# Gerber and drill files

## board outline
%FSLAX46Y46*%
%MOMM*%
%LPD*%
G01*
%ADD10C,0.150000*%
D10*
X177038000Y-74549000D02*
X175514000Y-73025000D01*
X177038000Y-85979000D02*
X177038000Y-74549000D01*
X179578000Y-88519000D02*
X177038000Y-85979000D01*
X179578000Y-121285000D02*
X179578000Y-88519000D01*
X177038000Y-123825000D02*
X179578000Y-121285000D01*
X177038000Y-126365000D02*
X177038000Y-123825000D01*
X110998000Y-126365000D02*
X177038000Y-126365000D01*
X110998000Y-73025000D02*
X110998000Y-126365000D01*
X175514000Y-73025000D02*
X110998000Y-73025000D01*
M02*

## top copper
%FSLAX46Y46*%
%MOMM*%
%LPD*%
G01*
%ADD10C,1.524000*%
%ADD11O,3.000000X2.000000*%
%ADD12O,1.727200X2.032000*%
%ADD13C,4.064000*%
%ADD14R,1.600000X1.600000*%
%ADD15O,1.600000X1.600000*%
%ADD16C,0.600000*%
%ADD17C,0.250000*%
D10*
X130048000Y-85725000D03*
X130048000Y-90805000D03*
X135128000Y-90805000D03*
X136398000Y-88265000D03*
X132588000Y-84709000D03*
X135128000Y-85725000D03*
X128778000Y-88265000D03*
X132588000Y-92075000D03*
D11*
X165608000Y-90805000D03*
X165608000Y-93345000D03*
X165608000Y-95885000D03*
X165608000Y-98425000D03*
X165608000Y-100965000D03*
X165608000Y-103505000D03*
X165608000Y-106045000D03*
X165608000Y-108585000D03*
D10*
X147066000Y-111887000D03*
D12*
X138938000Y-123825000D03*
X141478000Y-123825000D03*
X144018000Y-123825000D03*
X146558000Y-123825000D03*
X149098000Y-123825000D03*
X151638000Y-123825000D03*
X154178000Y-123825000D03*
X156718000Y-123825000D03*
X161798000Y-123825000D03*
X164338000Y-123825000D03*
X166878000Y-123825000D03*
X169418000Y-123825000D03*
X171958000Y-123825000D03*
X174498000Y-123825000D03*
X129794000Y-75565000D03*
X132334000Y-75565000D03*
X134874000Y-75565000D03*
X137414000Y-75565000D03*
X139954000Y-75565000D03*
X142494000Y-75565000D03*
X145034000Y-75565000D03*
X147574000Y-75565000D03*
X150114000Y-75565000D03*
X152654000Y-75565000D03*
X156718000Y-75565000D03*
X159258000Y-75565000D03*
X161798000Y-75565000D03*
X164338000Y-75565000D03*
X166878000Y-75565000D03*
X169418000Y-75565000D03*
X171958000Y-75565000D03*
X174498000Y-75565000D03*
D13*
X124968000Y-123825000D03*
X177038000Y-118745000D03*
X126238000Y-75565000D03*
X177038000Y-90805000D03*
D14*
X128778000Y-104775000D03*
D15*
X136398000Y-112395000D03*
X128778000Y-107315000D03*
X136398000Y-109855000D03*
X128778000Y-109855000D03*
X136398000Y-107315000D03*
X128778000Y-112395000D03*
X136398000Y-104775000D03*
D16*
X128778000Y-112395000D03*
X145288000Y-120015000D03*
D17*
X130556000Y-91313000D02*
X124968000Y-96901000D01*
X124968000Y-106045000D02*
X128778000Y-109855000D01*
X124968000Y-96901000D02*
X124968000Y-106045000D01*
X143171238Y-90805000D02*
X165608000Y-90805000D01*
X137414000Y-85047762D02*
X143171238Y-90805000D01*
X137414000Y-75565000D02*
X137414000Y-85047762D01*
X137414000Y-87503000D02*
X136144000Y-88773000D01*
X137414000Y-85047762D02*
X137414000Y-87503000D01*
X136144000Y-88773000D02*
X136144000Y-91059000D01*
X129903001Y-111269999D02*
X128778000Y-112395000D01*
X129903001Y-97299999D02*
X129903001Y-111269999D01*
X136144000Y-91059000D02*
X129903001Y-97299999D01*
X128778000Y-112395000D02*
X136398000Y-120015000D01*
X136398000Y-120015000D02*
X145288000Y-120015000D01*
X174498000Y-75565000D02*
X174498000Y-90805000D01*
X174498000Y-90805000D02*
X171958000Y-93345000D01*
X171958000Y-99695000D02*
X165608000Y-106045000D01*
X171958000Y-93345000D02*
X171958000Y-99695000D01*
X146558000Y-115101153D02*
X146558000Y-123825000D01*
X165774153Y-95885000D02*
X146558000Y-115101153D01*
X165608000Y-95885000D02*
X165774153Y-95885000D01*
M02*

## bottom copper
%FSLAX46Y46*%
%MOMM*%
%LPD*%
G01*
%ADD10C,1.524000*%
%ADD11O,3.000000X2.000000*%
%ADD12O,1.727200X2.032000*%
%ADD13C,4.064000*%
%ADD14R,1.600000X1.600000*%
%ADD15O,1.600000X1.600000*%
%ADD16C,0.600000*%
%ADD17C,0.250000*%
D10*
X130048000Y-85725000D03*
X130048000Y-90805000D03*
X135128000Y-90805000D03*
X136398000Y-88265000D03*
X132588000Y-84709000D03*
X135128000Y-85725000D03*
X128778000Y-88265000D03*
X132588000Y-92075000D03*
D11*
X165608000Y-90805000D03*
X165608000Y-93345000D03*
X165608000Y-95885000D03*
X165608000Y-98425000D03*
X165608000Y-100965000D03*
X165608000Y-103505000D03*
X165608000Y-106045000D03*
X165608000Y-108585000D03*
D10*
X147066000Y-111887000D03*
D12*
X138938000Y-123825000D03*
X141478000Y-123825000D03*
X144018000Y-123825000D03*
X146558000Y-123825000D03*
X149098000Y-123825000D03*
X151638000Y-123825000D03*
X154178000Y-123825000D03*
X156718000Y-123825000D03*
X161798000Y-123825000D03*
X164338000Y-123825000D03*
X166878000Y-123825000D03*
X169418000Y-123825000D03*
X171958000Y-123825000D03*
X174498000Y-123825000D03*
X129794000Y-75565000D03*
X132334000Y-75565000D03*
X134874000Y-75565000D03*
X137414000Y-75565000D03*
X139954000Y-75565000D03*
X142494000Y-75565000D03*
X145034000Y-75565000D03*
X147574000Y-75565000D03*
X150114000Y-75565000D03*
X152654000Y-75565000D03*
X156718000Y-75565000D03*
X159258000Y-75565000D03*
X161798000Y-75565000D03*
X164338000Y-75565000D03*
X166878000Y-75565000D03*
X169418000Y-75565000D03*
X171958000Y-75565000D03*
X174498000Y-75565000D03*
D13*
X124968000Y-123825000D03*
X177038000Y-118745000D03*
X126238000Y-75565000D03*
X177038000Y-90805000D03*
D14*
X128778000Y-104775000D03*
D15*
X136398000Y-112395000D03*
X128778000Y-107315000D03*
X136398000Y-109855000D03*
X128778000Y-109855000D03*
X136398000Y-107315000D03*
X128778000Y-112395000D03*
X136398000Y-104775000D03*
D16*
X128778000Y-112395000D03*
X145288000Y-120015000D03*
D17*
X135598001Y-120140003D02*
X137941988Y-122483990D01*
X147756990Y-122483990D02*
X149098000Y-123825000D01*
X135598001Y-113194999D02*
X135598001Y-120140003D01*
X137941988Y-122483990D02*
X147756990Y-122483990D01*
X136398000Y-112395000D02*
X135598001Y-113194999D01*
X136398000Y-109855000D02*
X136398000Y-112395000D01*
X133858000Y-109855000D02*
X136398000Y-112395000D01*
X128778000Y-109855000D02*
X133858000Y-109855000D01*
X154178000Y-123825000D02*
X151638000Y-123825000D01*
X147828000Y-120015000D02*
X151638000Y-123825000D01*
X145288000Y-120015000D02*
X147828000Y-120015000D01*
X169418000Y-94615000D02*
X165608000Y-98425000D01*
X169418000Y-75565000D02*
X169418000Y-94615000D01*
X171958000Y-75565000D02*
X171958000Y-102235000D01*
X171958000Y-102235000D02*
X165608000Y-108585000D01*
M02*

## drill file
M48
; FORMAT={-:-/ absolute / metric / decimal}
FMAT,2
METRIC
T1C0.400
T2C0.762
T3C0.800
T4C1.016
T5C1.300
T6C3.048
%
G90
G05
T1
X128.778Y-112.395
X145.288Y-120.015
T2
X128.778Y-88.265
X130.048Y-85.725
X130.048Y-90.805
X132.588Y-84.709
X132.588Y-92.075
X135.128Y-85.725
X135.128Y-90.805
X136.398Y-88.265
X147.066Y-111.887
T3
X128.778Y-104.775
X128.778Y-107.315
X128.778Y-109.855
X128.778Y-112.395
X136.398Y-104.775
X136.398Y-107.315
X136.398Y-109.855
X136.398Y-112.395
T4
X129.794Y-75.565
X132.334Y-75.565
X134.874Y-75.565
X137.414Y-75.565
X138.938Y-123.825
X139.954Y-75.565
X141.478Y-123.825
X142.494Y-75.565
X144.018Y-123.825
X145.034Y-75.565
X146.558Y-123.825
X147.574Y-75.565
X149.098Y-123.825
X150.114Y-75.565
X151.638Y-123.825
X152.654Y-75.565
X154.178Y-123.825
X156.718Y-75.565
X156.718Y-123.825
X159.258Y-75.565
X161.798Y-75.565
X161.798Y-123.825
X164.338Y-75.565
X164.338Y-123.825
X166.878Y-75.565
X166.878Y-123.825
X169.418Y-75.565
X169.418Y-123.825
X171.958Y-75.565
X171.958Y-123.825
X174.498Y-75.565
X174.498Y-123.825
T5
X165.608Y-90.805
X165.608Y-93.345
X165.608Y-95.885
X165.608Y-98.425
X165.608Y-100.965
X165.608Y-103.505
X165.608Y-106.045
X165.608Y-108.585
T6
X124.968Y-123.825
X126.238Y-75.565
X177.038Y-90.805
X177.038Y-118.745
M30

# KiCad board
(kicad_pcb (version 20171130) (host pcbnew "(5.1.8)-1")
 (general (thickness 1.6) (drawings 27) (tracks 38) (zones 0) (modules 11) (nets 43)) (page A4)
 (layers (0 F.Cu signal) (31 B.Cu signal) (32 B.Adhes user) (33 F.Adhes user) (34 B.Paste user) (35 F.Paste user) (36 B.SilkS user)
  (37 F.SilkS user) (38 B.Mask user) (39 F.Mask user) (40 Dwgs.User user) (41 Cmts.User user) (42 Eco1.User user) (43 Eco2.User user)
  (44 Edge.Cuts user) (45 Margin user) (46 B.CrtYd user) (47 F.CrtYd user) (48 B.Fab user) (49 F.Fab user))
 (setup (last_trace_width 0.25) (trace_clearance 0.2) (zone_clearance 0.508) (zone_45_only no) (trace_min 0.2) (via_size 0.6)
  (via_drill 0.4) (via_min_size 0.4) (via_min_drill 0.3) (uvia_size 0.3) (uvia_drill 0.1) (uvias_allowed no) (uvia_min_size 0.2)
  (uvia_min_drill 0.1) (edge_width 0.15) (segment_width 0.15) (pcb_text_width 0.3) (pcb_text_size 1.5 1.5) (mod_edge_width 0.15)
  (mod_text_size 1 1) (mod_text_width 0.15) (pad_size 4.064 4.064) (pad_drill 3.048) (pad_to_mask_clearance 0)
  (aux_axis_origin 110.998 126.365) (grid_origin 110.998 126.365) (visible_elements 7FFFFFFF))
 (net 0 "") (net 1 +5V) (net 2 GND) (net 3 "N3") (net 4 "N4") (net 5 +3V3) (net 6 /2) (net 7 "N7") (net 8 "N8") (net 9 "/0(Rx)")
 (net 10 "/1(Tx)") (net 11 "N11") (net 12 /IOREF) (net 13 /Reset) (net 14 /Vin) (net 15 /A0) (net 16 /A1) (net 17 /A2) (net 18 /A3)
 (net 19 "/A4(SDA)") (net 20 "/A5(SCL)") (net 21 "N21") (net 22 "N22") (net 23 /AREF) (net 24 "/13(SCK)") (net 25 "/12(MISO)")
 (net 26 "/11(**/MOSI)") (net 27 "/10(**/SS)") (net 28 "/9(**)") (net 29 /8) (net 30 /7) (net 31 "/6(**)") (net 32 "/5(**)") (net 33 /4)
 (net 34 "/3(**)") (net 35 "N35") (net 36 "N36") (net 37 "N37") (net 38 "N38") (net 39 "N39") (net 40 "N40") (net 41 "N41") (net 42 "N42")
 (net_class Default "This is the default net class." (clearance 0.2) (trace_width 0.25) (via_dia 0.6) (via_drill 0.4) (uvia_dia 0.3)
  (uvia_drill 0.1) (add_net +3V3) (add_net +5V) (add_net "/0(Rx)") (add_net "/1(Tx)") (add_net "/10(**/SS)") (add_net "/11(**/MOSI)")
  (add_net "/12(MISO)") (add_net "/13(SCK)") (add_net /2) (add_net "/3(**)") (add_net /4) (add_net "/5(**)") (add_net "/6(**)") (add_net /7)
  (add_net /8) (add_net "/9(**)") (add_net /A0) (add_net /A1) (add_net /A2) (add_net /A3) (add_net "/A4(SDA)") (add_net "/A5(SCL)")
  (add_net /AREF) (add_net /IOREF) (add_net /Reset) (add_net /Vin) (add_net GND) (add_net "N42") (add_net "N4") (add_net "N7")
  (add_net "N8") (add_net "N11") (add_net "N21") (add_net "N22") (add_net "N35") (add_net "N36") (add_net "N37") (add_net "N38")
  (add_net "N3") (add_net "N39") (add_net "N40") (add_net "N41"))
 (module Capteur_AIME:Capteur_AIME (layer F.Cu) (at 132.588 88.265)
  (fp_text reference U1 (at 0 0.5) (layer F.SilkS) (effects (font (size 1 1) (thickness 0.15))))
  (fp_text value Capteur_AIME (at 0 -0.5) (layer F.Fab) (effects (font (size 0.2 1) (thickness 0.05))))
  (pad 2 thru_hole circle (at -2.54 -2.54) (size 1.524 1.524) (drill 0.762) (layers *.Cu *.Mask) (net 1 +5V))
  (pad 8 thru_hole circle (at -2.54 2.54) (size 1.524 1.524) (drill 0.762) (layers *.Cu *.Mask))
  (pad 6 thru_hole circle (at 2.54 2.54) (size 1.524 1.524) (drill 0.762) (layers *.Cu *.Mask))
  (pad 5 thru_hole circle (at 3.81 0) (size 1.524 1.524) (drill 0.762) (layers *.Cu *.Mask) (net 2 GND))
  (pad 3 thru_hole circle (at 0 -3.556) (size 1.524 1.524) (drill 0.762) (layers *.Cu *.Mask) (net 1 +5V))
  (pad 4 thru_hole circle (at 2.54 -2.54) (size 1.524 1.524) (drill 0.762) (layers *.Cu *.Mask) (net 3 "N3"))
  (pad 1 thru_hole circle (at -3.81 0) (size 1.524 1.524) (drill 0.762) (layers *.Cu *.Mask))
  (pad 7 thru_hole circle (at 0 3.81) (size 1.524 1.524) (drill 0.762) (layers *.Cu *.Mask)))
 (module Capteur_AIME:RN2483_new (layer F.Cu) (at 165.608 99.695 270)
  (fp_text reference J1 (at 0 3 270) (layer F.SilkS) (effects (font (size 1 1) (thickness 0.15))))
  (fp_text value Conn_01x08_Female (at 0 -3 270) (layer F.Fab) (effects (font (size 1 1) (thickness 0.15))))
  (pad 1 thru_hole oval (at -8.89 0 270) (size 2 3) (drill 1.3) (layers *.Cu *.Mask) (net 2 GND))
  (pad 2 thru_hole oval (at -6.35 0 270) (size 2 3) (drill 1.3) (layers *.Cu *.Mask) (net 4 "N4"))
  (pad 3 thru_hole oval (at -3.81 0 270) (size 2 3) (drill 1.3) (layers *.Cu *.Mask) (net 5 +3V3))
  (pad 4 thru_hole oval (at -1.27 0 270) (size 2 3) (drill 1.3) (layers *.Cu *.Mask) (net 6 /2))
  (pad 5 thru_hole oval (at 1.27 0 270) (size 2 3) (drill 1.3) (layers *.Cu *.Mask) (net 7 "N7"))
  (pad 6 thru_hole oval (at 3.81 0 270) (size 2 3) (drill 1.3) (layers *.Cu *.Mask) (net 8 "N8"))
  (pad 7 thru_hole oval (at 6.35 0 270) (size 2 3) (drill 1.3) (layers *.Cu *.Mask) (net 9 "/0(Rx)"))
  (pad 8 thru_hole oval (at 8.89 0 270) (size 2 3) (drill 1.3) (layers *.Cu *.Mask) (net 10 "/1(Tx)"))
  (pad 9 thru_hole circle (at 12.192 18.542 270) (size 1.524 1.524) (drill 0.762) (layers *.Cu *.Mask)))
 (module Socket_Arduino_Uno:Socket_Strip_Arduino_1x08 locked (layer F.Cu) (at 138.938 123.825)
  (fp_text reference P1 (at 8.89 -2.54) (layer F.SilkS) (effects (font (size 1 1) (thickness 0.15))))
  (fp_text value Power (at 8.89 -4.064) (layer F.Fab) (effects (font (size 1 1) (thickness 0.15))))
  (pad 1 thru_hole oval (at 0 0) (size 1.7272 2.032) (drill 1.016) (layers *.Cu *.Mask F.SilkS) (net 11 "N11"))
  (pad 2 thru_hole oval (at 2.54 0) (size 1.7272 2.032) (drill 1.016) (layers *.Cu *.Mask F.SilkS) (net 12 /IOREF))
  (pad 3 thru_hole oval (at 5.08 0) (size 1.7272 2.032) (drill 1.016) (layers *.Cu *.Mask F.SilkS) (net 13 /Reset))
  (pad 4 thru_hole oval (at 7.62 0) (size 1.7272 2.032) (drill 1.016) (layers *.Cu *.Mask F.SilkS) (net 5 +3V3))
  (pad 5 thru_hole oval (at 10.16 0) (size 1.7272 2.032) (drill 1.016) (layers *.Cu *.Mask F.SilkS) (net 1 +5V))
  (pad 6 thru_hole oval (at 12.7 0) (size 1.7272 2.032) (drill 1.016) (layers *.Cu *.Mask F.SilkS) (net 2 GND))
  (pad 7 thru_hole oval (at 15.24 0) (size 1.7272 2.032) (drill 1.016) (layers *.Cu *.Mask F.SilkS) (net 2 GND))
  (pad 8 thru_hole oval (at 17.78 0) (size 1.7272 2.032) (drill 1.016) (layers *.Cu *.Mask F.SilkS) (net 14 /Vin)))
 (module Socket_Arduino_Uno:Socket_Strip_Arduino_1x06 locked (layer F.Cu) (at 161.798 123.825)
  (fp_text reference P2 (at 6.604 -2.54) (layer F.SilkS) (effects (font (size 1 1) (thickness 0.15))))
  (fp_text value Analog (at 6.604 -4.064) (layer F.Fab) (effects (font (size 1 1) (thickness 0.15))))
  (pad 1 thru_hole oval (at 0 0) (size 1.7272 2.032) (drill 1.016) (layers *.Cu *.Mask F.SilkS) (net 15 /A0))
  (pad 2 thru_hole oval (at 2.54 0) (size 1.7272 2.032) (drill 1.016) (layers *.Cu *.Mask F.SilkS) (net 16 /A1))
  (pad 3 thru_hole oval (at 5.08 0) (size 1.7272 2.032) (drill 1.016) (layers *.Cu *.Mask F.SilkS) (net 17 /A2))
  (pad 4 thru_hole oval (at 7.62 0) (size 1.7272 2.032) (drill 1.016) (layers *.Cu *.Mask F.SilkS) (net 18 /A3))
  (pad 5 thru_hole oval (at 10.16 0) (size 1.7272 2.032) (drill 1.016) (layers *.Cu *.Mask F.SilkS) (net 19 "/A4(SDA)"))
  (pad 6 thru_hole oval (at 12.7 0) (size 1.7272 2.032) (drill 1.016) (layers *.Cu *.Mask F.SilkS) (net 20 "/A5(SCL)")))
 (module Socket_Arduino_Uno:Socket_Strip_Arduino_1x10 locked (layer F.Cu) (at 129.794 75.565)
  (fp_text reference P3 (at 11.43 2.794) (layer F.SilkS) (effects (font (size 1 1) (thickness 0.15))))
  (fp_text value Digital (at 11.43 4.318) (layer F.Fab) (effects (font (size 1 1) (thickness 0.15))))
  (pad 1 thru_hole oval (at 0 0) (size 1.7272 2.032) (drill 1.016) (layers *.Cu *.Mask F.SilkS) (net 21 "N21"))
  (pad 2 thru_hole oval (at 2.54 0) (size 1.7272 2.032) (drill 1.016) (layers *.Cu *.Mask F.SilkS) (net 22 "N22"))
  (pad 3 thru_hole oval (at 5.08 0) (size 1.7272 2.032) (drill 1.016) (layers *.Cu *.Mask F.SilkS) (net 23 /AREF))
  (pad 4 thru_hole oval (at 7.62 0) (size 1.7272 2.032) (drill 1.016) (layers *.Cu *.Mask F.SilkS) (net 2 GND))
  (pad 5 thru_hole oval (at 10.16 0) (size 1.7272 2.032) (drill 1.016) (layers *.Cu *.Mask F.SilkS) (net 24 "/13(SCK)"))
  (pad 6 thru_hole oval (at 12.7 0) (size 1.7272 2.032) (drill 1.016) (layers *.Cu *.Mask F.SilkS) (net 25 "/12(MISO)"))
  (pad 7 thru_hole oval (at 15.24 0) (size 1.7272 2.032) (drill 1.016) (layers *.Cu *.Mask F.SilkS) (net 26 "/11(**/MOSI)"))
  (pad 8 thru_hole oval (at 17.78 0) (size 1.7272 2.032) (drill 1.016) (layers *.Cu *.Mask F.SilkS) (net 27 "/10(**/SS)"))
  (pad 9 thru_hole oval (at 20.32 0) (size 1.7272 2.032) (drill 1.016) (layers *.Cu *.Mask F.SilkS) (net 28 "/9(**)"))
  (pad 10 thru_hole oval (at 22.86 0) (size 1.7272 2.032) (drill 1.016) (layers *.Cu *.Mask F.SilkS) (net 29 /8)))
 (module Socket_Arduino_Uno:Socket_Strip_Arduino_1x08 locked (layer F.Cu) (at 156.718 75.565)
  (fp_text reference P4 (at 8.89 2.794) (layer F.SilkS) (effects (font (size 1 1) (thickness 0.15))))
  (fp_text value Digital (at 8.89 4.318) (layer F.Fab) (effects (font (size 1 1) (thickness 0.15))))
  (pad 1 thru_hole oval (at 0 0) (size 1.7272 2.032) (drill 1.016) (layers *.Cu *.Mask F.SilkS) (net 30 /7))
  (pad 2 thru_hole oval (at 2.54 0) (size 1.7272 2.032) (drill 1.016) (layers *.Cu *.Mask F.SilkS) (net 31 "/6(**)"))
  (pad 3 thru_hole oval (at 5.08 0) (size 1.7272 2.032) (drill 1.016) (layers *.Cu *.Mask F.SilkS) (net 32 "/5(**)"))
  (pad 4 thru_hole oval (at 7.62 0) (size 1.7272 2.032) (drill 1.016) (layers *.Cu *.Mask F.SilkS) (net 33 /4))
  (pad 5 thru_hole oval (at 10.16 0) (size 1.7272 2.032) (drill 1.016) (layers *.Cu *.Mask F.SilkS) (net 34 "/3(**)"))
  (pad 6 thru_hole oval (at 12.7 0) (size 1.7272 2.032) (drill 1.016) (layers *.Cu *.Mask F.SilkS) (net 6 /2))
  (pad 7 thru_hole oval (at 15.24 0) (size 1.7272 2.032) (drill 1.016) (layers *.Cu *.Mask F.SilkS) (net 10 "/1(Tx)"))
  (pad 8 thru_hole oval (at 17.78 0) (size 1.7272 2.032) (drill 1.016) (layers *.Cu *.Mask F.SilkS) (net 9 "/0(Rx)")))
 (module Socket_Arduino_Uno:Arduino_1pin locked (layer F.Cu) (at 124.968 123.825)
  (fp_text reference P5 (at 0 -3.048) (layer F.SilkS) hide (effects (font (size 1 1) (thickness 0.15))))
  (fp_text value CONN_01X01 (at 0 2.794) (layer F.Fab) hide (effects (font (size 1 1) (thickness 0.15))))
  (pad 1 thru_hole circle (at 0 0) (size 4.064 4.064) (drill 3.048) (layers *.Cu *.Mask F.SilkS) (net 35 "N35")))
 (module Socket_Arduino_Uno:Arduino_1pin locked (layer F.Cu) (at 177.038 118.745)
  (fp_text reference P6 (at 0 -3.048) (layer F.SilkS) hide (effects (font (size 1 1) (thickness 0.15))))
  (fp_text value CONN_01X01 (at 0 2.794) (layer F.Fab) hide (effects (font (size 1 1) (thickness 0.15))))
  (pad 1 thru_hole circle (at 0 0) (size 4.064 4.064) (drill 3.048) (layers *.Cu *.Mask F.SilkS) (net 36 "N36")))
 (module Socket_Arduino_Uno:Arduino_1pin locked (layer F.Cu) (at 126.238 75.565)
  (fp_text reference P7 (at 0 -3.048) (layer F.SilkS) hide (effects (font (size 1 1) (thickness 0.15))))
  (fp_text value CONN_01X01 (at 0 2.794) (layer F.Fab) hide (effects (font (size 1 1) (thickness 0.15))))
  (pad 1 thru_hole circle (at 0 0) (size 4.064 4.064) (drill 3.048) (layers *.Cu *.Mask F.SilkS) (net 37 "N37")))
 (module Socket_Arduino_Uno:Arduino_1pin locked (layer F.Cu) (at 177.038 90.805)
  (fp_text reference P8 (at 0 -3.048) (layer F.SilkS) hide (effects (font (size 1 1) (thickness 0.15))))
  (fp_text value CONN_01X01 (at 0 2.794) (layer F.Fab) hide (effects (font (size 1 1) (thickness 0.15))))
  (pad 1 thru_hole circle (at 0 0) (size 4.064 4.064) (drill 3.048) (layers *.Cu *.Mask F.SilkS) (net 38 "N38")))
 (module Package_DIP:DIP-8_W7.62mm (layer F.Cu) (at 128.778 104.775)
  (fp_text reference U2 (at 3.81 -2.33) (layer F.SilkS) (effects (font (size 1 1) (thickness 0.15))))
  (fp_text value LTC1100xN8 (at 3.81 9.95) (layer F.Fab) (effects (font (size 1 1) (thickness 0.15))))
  (pad 1 thru_hole rect (at 0 0) (size 1.6 1.6) (drill 0.8) (layers *.Cu *.Mask) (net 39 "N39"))
  (pad 5 thru_hole oval (at 7.62 7.62) (size 1.6 1.6) (drill 0.8) (layers *.Cu *.Mask) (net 1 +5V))
  (pad 2 thru_hole oval (at 0 2.54) (size 1.6 1.6) (drill 0.8) (layers *.Cu *.Mask) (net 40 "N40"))
  (pad 6 thru_hole oval (at 7.62 5.08) (size 1.6 1.6) (drill 0.8) (layers *.Cu *.Mask) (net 1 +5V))
  (pad 3 thru_hole oval (at 0 5.08) (size 1.6 1.6) (drill 0.8) (layers *.Cu *.Mask) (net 1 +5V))
  (pad 7 thru_hole oval (at 7.62 2.54) (size 1.6 1.6) (drill 0.8) (layers *.Cu *.Mask) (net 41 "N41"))
  (pad 4 thru_hole oval (at 0 7.62) (size 1.6 1.6) (drill 0.8) (layers *.Cu *.Mask) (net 2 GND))
  (pad 8 thru_hole oval (at 7.62 0) (size 1.6 1.6) (drill 0.8) (layers *.Cu *.Mask) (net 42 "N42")))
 (gr_line (start 177.038 74.549) (end 175.514 73.025) (angle 90) (layer Edge.Cuts) (width 0.15))
 (gr_line (start 177.038 85.979) (end 177.038 74.549) (angle 90) (layer Edge.Cuts) (width 0.15))
 (gr_line (start 179.578 88.519) (end 177.038 85.979) (angle 90) (layer Edge.Cuts) (width 0.15))
 (gr_line (start 179.578 121.285) (end 179.578 88.519) (angle 90) (layer Edge.Cuts) (width 0.15))
 (gr_line (start 177.038 123.825) (end 179.578 121.285) (angle 90) (layer Edge.Cuts) (width 0.15))
 (gr_line (start 177.038 126.365) (end 177.038 123.825) (angle 90) (layer Edge.Cuts) (width 0.15))
 (gr_line (start 110.998 126.365) (end 177.038 126.365) (angle 90) (layer Edge.Cuts) (width 0.15))
 (gr_line (start 110.998 73.025) (end 110.998 126.365) (angle 90) (layer Edge.Cuts) (width 0.15))
 (gr_line (start 175.514 73.025) (end 110.998 73.025) (angle 90) (layer Edge.Cuts) (width 0.15))
 (segment (start 130.556 91.313) (end 124.968 96.901) (width 0.25) (layer F.Cu) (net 1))
 (segment (start 124.968 106.045) (end 128.778 109.855) (width 0.25) (layer F.Cu) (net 1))
 (segment (start 124.968 96.901) (end 124.968 106.045) (width 0.25) (layer F.Cu) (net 1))
 (segment (start 135.598001 120.140003) (end 137.941988 122.48399) (width 0.25) (layer B.Cu) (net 1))
 (segment (start 147.75699 122.48399) (end 149.098 123.825) (width 0.25) (layer B.Cu) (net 1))
 (segment (start 135.598001 113.194999) (end 135.598001 120.140003) (width 0.25) (layer B.Cu) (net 1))
 (segment (start 137.941988 122.48399) (end 147.75699 122.48399) (width 0.25) (layer B.Cu) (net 1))
 (segment (start 136.398 112.395) (end 135.598001 113.194999) (width 0.25) (layer B.Cu) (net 1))
 (segment (start 136.398 109.855) (end 136.398 112.395) (width 0.25) (layer B.Cu) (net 1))
 (segment (start 133.858 109.855) (end 136.398 112.395) (width 0.25) (layer B.Cu) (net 1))
 (segment (start 128.778 109.855) (end 133.858 109.855) (width 0.25) (layer B.Cu) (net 1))
 (segment (start 143.171238 90.805) (end 165.608 90.805) (width 0.25) (layer F.Cu) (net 2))
 (segment (start 137.414 85.047762) (end 143.171238 90.805) (width 0.25) (layer F.Cu) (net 2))
 (segment (start 137.414 75.565) (end 137.414 85.047762) (width 0.25) (layer F.Cu) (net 2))
 (segment (start 137.414 87.503) (end 136.144 88.773) (width 0.25) (layer F.Cu) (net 2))
 (segment (start 137.414 85.047762) (end 137.414 87.503) (width 0.25) (layer F.Cu) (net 2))
 (segment (start 136.144 88.773) (end 136.144 91.059) (width 0.25) (layer F.Cu) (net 2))
 (via (at 128.778 112.395) (size 0.6) (drill 0.4) (layers F.Cu B.Cu) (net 2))
 (segment (start 129.903001 111.269999) (end 128.778 112.395) (width 0.25) (layer F.Cu) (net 2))
 (segment (start 129.903001 97.299999) (end 129.903001 111.269999) (width 0.25) (layer F.Cu) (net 2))
 (segment (start 136.144 91.059) (end 129.903001 97.299999) (width 0.25) (layer F.Cu) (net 2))
 (segment (start 154.178 123.825) (end 151.638 123.825) (width 0.25) (layer B.Cu) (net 2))
 (segment (start 128.778 112.395) (end 136.398 120.015) (width 0.25) (layer F.Cu) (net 2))
 (via (at 145.288 120.015) (size 0.6) (drill 0.4) (layers F.Cu B.Cu) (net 2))
 (segment (start 136.398 120.015) (end 145.288 120.015) (width 0.25) (layer F.Cu) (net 2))
 (segment (start 147.828 120.015) (end 151.638 123.825) (width 0.25) (layer B.Cu) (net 2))
 (segment (start 145.288 120.015) (end 147.828 120.015) (width 0.25) (layer B.Cu) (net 2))
 (segment (start 169.418 94.615) (end 165.608 98.425) (width 0.25) (layer B.Cu) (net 6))
 (segment (start 169.418 75.565) (end 169.418 94.615) (width 0.25) (layer B.Cu) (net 6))
 (segment (start 171.958 75.565) (end 171.958 102.235) (width 0.25) (layer B.Cu) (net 10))
 (segment (start 171.958 102.235) (end 165.608 108.585) (width 0.25) (layer B.Cu) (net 10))
 (segment (start 174.498 75.565) (end 174.498 90.805) (width 0.25) (layer F.Cu) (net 9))
 (segment (start 174.498 90.805) (end 171.958 93.345) (width 0.25) (layer F.Cu) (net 9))
 (segment (start 171.958 99.695) (end 165.608 106.045) (width 0.25) (layer F.Cu) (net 9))
 (segment (start 171.958 93.345) (end 171.958 99.695) (width 0.25) (layer F.Cu) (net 9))
 (segment (start 146.558 115.101153) (end 146.558 123.825) (width 0.25) (layer F.Cu) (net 5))
 (segment (start 165.774153 95.885) (end 146.558 115.101153) (width 0.25) (layer F.Cu) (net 5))
 (segment (start 165.608 95.885) (end 165.774153 95.885) (width 0.25) (layer F.Cu) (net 5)))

